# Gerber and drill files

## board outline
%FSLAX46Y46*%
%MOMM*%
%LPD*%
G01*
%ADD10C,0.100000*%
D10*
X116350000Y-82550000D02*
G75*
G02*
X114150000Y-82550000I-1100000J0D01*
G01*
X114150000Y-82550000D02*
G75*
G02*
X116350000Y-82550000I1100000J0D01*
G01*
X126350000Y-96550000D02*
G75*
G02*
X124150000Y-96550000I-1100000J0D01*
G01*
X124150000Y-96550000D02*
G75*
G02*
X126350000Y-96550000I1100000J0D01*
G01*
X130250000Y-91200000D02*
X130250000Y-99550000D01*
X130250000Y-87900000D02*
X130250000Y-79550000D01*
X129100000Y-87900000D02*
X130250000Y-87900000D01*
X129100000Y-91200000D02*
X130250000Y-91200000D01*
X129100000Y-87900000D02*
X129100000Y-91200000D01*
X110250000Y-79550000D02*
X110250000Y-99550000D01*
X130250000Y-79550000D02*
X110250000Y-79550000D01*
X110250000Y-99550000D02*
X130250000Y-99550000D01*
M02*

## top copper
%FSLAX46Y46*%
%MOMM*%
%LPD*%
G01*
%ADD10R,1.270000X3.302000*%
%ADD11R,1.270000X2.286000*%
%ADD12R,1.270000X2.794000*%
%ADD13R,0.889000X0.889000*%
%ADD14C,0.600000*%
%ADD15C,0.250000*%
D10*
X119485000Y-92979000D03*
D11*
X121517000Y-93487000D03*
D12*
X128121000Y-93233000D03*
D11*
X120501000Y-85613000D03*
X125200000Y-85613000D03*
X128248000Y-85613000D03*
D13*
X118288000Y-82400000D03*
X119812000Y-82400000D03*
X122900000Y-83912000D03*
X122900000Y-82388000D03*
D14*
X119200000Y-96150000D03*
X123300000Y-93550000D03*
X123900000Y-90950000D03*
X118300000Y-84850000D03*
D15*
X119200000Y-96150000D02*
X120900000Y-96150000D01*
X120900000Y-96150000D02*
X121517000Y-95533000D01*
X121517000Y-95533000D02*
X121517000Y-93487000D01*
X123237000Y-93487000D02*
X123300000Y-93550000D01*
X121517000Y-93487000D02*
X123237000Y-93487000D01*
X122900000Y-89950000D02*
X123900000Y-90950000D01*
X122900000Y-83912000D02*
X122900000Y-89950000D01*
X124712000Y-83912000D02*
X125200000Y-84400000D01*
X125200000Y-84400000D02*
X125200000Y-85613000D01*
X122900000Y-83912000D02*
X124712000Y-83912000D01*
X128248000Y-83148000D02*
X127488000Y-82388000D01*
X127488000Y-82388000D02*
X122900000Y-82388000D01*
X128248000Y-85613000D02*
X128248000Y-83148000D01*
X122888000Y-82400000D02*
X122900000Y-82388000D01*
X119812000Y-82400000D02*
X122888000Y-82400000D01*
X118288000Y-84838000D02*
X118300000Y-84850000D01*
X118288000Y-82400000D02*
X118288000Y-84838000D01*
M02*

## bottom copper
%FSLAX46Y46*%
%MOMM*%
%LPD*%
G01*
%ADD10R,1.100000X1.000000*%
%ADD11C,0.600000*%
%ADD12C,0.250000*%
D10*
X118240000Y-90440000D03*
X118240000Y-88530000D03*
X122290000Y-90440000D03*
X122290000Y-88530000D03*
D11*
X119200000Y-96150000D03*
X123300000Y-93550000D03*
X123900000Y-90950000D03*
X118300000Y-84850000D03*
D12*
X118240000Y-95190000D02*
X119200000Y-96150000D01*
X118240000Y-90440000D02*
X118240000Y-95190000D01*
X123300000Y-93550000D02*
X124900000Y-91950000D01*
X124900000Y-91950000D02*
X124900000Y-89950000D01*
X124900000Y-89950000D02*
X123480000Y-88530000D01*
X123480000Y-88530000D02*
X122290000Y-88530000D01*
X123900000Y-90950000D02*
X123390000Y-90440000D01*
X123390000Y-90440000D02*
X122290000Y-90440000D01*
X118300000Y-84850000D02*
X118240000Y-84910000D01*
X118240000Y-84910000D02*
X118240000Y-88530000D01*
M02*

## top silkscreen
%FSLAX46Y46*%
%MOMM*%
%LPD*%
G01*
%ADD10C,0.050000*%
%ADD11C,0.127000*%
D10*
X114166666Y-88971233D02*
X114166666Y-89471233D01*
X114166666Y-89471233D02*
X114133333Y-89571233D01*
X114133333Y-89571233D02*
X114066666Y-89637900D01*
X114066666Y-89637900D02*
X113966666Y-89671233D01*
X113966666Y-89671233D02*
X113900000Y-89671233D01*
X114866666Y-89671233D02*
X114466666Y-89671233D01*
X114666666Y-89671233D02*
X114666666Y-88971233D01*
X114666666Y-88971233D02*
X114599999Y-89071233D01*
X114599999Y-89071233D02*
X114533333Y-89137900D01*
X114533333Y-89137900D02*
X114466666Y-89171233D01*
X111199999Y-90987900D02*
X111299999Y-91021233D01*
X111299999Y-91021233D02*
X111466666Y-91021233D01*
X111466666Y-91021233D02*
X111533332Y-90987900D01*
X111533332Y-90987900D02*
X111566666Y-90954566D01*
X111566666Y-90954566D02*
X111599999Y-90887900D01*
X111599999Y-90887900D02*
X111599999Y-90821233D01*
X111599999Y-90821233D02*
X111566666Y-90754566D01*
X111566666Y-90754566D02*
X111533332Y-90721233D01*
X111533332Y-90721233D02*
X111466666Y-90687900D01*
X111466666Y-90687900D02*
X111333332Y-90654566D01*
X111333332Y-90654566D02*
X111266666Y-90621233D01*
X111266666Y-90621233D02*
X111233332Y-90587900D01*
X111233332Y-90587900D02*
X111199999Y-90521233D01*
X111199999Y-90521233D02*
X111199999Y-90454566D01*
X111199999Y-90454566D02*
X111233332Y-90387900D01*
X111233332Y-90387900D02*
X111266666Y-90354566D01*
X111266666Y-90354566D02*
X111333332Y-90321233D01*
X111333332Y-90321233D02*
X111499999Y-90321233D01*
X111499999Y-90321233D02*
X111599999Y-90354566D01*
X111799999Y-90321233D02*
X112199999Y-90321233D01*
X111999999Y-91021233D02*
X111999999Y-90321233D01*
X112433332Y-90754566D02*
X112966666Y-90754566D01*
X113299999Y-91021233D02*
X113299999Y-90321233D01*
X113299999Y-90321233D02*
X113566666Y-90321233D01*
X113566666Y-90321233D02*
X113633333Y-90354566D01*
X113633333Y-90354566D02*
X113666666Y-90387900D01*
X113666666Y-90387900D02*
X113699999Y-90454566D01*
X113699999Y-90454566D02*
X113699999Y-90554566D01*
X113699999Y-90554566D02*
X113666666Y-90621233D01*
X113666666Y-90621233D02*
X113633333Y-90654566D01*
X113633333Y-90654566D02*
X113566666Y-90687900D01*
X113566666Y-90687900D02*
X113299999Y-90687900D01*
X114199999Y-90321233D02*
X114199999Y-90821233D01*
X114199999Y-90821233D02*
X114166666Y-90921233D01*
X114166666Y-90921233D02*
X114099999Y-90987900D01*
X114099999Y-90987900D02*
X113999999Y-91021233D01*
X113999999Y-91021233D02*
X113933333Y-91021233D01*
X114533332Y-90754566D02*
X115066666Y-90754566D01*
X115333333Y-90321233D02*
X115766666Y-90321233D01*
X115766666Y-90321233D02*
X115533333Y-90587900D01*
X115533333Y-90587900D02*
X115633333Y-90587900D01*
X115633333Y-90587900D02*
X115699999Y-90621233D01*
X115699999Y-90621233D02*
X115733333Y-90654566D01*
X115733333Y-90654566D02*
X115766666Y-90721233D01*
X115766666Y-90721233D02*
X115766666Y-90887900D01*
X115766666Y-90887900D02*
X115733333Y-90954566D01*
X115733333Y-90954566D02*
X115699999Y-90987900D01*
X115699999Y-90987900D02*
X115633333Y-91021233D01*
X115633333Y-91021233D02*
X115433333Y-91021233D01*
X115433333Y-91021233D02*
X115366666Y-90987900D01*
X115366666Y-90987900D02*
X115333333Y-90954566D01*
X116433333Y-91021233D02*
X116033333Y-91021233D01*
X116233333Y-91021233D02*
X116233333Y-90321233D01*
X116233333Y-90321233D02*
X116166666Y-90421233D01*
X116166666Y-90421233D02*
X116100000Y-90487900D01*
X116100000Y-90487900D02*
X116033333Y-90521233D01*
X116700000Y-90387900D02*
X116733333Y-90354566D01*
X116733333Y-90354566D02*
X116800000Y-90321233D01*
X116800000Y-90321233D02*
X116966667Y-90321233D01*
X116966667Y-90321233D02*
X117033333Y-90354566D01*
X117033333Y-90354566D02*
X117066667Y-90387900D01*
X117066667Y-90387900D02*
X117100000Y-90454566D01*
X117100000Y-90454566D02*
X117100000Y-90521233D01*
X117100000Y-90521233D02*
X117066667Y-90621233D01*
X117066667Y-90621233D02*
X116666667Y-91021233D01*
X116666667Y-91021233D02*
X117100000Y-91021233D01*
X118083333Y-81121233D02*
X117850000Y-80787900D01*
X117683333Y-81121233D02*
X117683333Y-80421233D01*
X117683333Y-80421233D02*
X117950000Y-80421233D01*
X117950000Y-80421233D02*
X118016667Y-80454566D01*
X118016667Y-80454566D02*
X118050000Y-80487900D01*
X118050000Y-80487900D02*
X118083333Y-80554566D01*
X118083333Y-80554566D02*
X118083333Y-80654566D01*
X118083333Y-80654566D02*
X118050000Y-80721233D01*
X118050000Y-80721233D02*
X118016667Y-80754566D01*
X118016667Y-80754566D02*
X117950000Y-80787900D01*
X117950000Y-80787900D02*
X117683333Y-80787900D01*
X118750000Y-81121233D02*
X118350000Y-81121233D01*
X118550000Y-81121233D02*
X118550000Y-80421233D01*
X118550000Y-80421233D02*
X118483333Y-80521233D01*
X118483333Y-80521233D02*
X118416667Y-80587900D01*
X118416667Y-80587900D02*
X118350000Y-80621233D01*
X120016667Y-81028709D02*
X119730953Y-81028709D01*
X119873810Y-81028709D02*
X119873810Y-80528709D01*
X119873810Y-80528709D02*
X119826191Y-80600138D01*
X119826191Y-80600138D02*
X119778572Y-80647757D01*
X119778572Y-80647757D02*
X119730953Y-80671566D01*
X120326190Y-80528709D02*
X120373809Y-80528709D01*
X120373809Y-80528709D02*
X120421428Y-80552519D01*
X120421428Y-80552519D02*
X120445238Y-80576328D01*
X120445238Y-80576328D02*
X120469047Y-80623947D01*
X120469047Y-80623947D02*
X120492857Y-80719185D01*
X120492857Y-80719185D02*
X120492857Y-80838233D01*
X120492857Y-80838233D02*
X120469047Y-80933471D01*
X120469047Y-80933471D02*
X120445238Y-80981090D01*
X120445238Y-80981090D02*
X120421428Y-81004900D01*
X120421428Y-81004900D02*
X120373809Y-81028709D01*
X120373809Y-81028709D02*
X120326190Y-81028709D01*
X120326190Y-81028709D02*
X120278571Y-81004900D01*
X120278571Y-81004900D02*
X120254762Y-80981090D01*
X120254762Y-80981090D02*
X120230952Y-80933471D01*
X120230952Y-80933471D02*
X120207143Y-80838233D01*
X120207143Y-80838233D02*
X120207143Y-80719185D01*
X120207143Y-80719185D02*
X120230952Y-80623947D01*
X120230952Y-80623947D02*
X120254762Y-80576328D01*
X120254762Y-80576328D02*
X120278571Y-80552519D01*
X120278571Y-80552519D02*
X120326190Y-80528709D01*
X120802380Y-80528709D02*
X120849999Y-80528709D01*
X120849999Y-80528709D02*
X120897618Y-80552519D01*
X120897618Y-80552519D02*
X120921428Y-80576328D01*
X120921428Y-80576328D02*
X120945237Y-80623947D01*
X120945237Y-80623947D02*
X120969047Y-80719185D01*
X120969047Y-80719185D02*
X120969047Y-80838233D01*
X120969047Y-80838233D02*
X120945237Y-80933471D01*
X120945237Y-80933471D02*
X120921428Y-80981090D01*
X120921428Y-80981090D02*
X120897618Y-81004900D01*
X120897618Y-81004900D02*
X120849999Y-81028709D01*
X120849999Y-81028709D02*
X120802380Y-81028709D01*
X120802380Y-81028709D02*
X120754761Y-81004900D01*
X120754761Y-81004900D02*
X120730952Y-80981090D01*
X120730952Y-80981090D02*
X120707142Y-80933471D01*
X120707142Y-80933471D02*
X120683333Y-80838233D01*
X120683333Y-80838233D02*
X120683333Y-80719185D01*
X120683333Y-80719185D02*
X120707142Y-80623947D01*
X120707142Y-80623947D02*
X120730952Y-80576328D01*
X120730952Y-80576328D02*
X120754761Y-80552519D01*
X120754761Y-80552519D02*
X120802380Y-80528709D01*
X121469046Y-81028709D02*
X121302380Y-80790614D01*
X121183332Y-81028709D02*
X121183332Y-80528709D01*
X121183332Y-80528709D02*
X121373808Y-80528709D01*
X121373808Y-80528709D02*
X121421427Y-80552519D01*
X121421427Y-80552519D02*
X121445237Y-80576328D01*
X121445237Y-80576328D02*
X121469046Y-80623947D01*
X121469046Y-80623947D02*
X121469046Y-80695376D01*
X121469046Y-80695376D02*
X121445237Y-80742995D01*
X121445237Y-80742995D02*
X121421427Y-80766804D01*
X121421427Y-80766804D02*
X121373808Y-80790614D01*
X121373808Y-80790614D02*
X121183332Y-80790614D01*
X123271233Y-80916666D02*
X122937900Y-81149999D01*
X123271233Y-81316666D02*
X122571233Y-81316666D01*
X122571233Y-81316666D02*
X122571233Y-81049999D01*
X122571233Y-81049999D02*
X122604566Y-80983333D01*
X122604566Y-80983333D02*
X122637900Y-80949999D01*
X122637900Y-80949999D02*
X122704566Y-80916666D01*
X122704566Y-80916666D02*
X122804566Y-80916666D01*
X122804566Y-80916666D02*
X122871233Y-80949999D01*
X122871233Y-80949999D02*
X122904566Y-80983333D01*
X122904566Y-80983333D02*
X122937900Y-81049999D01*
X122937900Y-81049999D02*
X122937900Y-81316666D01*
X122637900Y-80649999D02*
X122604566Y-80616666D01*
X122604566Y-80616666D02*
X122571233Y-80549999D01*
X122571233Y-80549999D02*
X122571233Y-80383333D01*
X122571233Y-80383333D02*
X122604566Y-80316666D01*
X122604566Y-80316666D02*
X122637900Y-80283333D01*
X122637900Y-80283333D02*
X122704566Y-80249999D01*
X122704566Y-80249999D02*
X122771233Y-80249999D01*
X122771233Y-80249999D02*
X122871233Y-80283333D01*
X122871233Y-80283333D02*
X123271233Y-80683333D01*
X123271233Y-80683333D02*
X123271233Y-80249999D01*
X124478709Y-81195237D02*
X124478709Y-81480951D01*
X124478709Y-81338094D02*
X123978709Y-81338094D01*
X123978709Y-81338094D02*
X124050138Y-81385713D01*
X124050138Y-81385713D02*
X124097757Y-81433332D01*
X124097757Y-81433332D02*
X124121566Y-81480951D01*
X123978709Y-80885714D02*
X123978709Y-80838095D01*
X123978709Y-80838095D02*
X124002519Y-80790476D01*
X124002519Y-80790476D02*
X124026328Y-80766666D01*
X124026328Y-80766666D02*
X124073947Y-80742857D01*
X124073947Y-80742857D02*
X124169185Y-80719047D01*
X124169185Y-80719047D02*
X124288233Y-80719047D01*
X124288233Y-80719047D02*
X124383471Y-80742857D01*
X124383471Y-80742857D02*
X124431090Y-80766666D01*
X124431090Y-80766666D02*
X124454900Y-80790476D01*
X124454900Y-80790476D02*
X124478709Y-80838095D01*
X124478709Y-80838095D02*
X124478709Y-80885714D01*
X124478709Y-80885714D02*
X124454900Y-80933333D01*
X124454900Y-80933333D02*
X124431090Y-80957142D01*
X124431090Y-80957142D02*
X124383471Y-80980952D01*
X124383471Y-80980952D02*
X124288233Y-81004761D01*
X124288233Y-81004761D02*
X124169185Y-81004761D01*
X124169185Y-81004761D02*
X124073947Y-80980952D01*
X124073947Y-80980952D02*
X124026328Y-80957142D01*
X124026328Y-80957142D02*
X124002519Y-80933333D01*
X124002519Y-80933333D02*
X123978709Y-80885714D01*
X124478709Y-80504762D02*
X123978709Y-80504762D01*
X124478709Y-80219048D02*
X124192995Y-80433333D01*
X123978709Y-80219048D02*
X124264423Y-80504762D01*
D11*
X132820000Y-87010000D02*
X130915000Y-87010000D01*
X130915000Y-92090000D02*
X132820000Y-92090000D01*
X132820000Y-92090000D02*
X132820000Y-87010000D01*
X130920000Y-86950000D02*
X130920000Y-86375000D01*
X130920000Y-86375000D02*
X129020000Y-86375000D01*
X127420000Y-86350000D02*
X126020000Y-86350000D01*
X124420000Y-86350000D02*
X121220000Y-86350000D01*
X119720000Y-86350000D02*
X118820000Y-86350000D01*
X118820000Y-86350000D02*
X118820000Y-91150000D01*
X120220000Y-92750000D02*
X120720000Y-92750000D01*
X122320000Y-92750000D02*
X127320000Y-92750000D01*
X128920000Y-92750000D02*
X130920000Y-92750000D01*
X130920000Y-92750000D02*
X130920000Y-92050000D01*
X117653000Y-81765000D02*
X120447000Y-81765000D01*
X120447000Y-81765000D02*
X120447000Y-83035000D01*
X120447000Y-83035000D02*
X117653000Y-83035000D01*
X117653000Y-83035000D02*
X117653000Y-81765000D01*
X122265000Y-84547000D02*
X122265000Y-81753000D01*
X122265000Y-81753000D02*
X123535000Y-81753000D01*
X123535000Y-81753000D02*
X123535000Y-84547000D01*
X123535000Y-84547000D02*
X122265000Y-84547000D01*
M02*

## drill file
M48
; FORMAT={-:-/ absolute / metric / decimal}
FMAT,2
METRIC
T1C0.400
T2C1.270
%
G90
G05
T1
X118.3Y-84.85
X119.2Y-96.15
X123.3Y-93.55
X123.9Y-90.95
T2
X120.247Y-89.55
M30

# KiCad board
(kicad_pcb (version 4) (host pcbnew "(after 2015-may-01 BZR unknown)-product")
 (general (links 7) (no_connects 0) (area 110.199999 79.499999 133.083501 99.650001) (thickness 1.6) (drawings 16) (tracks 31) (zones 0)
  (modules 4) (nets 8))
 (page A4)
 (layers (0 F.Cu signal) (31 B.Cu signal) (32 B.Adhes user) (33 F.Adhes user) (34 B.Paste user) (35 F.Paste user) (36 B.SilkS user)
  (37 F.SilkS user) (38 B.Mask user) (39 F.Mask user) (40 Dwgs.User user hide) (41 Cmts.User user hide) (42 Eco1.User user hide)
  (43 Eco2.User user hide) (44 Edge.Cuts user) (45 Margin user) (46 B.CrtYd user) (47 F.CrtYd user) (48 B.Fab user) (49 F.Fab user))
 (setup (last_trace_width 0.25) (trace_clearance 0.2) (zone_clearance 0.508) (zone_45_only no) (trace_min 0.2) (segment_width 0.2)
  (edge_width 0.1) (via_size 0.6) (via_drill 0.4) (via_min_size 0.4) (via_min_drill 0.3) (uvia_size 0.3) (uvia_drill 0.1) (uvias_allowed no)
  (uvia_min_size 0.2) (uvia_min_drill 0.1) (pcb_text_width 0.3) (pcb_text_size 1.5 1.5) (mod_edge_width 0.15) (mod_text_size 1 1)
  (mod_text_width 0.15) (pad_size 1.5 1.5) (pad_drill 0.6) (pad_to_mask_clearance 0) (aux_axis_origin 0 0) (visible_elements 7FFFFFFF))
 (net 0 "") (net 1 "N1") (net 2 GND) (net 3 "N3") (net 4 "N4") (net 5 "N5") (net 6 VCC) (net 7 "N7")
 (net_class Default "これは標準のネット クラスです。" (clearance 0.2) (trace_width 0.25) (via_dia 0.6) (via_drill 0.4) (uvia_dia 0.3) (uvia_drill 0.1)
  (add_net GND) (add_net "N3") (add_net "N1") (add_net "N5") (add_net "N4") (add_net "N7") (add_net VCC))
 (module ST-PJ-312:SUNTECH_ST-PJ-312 (layer F.Cu) (at 125.2 89.55) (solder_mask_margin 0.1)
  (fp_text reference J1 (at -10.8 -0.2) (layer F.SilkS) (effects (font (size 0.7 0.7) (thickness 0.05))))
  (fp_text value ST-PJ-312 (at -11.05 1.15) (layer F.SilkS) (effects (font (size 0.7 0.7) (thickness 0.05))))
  (fp_line (start 7.62 -2.54) (end 5.715 -2.54) (layer F.SilkS) (width 0.127))
  (fp_line (start 5.715 2.54) (end 7.62 2.54) (layer F.SilkS) (width 0.127))
  (fp_line (start 7.62 2.54) (end 7.62 -2.54) (layer F.SilkS) (width 0.127))
  (fp_line (start 5.72 -2.6) (end 5.72 -3.175) (layer F.SilkS) (width 0.127))
  (fp_line (start 5.72 -3.175) (end 3.82 -3.175) (layer F.SilkS) (width 0.127))
  (fp_line (start 2.22 -3.2) (end 0.82 -3.2) (layer F.SilkS) (width 0.127))
  (fp_line (start -0.78 -3.2) (end -3.98 -3.2) (layer F.SilkS) (width 0.127))
  (fp_line (start -5.48 -3.2) (end -6.38 -3.2) (layer F.SilkS) (width 0.127))
  (fp_line (start -6.38 -3.2) (end -6.38 1.6) (layer F.SilkS) (width 0.127))
  (fp_line (start -4.98 3.2) (end -4.48 3.2) (layer F.SilkS) (width 0.127))
  (fp_line (start -2.88 3.2) (end 2.12 3.2) (layer F.SilkS) (width 0.127))
  (fp_line (start 3.72 3.2) (end 5.72 3.2) (layer F.SilkS) (width 0.127))
  (fp_line (start 5.72 3.2) (end 5.72 2.5) (layer F.SilkS) (width 0.127))
  (pad LS smd rect (at -5.715 3.429 90) (size 3.302 1.27) (layers F.Cu F.Paste F.Mask) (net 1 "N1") (solder_mask_margin 0.2))
  (pad L smd rect (at -3.683 3.937 90) (size 2.286 1.27) (layers F.Cu F.Paste F.Mask) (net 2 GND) (solder_mask_margin 0.2))
  (pad COM2 smd rect (at 2.921 3.683 90) (size 2.794 1.27) (layers F.Cu F.Paste F.Mask) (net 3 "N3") (solder_mask_margin 0.2))
  (pad RS smd rect (at -4.699 -3.937 90) (size 2.286 1.27) (layers F.Cu F.Paste F.Mask) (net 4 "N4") (solder_mask_margin 0.2))
  (pad R smd rect (at 0 -3.937 90) (size 2.286 1.27) (layers F.Cu F.Paste F.Mask) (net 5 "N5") (solder_mask_margin 0.2))
  (pad COM1 smd rect (at 3.048 -3.937 90) (size 2.286 1.27) (layers F.Cu F.Paste F.Mask) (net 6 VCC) (solder_mask_margin 0.2))
  (pad Hole np_thru_hole circle (at -4.953 0) (size 1.27 1.27) (drill 1.27) (layers)))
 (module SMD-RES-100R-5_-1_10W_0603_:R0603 (layer F.Cu) (at 119.05 82.4 90) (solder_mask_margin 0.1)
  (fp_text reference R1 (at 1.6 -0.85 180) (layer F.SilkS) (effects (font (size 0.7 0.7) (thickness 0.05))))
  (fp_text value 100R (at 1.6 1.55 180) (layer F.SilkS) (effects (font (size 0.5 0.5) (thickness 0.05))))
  (fp_line (start 0.635 -1.397) (end 0.635 1.397) (layer F.SilkS) (width 0.127))
  (fp_line (start 0.635 1.397) (end -0.635 1.397) (layer F.SilkS) (width 0.127))
  (fp_line (start -0.635 1.397) (end -0.635 -1.397) (layer F.SilkS) (width 0.127))
  (fp_line (start -0.635 -1.397) (end 0.635 -1.397) (layer F.SilkS) (width 0.127))
  (pad 1 smd rect (at 0 -0.762) (size 0.889 0.889) (layers F.Cu F.Paste F.Mask) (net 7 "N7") (solder_mask_margin 0.2))
  (pad 2 smd rect (at 0 0.762) (size 0.889 0.889) (layers F.Cu F.Paste F.Mask) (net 6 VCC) (solder_mask_margin 0.2)))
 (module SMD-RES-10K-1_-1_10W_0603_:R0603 (layer F.Cu) (at 122.9 83.15 180) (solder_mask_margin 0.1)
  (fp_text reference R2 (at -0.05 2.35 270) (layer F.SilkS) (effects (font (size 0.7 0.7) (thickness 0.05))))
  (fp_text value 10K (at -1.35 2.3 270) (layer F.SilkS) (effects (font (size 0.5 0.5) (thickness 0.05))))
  (fp_line (start 0.635 -1.397) (end 0.635 1.397) (layer F.SilkS) (width 0.127))
  (fp_line (start 0.635 1.397) (end -0.635 1.397) (layer F.SilkS) (width 0.127))
  (fp_line (start -0.635 1.397) (end -0.635 -1.397) (layer F.SilkS) (width 0.127))
  (fp_line (start -0.635 -1.397) (end 0.635 -1.397) (layer F.SilkS) (width 0.127))
  (pad 1 smd rect (at 0 -0.762 90) (size 0.889 0.889) (layers F.Cu F.Paste F.Mask) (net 5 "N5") (solder_mask_margin 0.2))
  (pad 2 smd rect (at 0 0.762 90) (size 0.889 0.889) (layers F.Cu F.Paste F.Mask) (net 6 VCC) (solder_mask_margin 0.2)))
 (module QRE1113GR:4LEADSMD (layer B.Cu) (at 120.25 89.5) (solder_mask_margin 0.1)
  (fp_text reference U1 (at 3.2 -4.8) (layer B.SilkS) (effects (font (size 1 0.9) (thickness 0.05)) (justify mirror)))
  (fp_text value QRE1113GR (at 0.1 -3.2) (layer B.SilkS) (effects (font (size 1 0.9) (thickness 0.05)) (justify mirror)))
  (pad E smd rect (at -2.01 0.94 90) (size 1 1.1) (layers B.Cu B.Paste B.Mask) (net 2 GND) (solder_mask_margin 0.2))
  (pad A smd rect (at -2.01 -0.97 90) (size 1 1.1) (layers B.Cu B.Paste B.Mask) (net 7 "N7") (solder_mask_margin 0.2))
  (pad C smd rect (at 2.04 0.94 90) (size 1 1.1) (layers B.Cu B.Paste B.Mask) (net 5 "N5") (solder_mask_margin 0.2))
  (pad K smd rect (at 2.04 -0.97 90) (size 1 1.1) (layers B.Cu B.Paste B.Mask) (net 2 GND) (solder_mask_margin 0.2)))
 (gr_circle (center 115.25 82.55) (end 116.35 82.55) (layer Edge.Cuts) (width 0.1))
 (gr_circle (center 125.25 96.55) (end 126.35 96.55) (layer Edge.Cuts) (width 0.1))
 (gr_line (start 130.25 91.2) (end 130.25 99.55) (angle 90) (layer Edge.Cuts) (width 0.1))
 (gr_line (start 130.25 87.9) (end 130.25 79.55) (angle 90) (layer Edge.Cuts) (width 0.1))
 (gr_line (start 129.1 87.9) (end 130.25 87.9) (angle 90) (layer Edge.Cuts) (width 0.1))
 (gr_line (start 129.1 91.2) (end 130.25 91.2) (angle 90) (layer Edge.Cuts) (width 0.1))
 (gr_line (start 129.1 87.9) (end 129.1 91.2) (angle 90) (layer Edge.Cuts) (width 0.1))
 (gr_line (start 110.25 79.55) (end 110.25 99.55) (angle 90) (layer Edge.Cuts) (width 0.1))
 (gr_line (start 130.25 79.55) (end 110.25 79.55) (angle 90) (layer Edge.Cuts) (width 0.1))
 (gr_line (start 110.25 99.55) (end 130.25 99.55) (angle 90) (layer Edge.Cuts) (width 0.1))
 (segment (start 118.24 95.19) (end 119.2 96.15) (width 0.25) (layer B.Cu) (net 2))
 (via (at 119.2 96.15) (size 0.6) (layers F.Cu B.Cu) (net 2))
 (segment (start 119.2 96.15) (end 120.9 96.15) (width 0.25) (layer F.Cu) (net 2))
 (segment (start 120.9 96.15) (end 121.517 95.533) (width 0.25) (layer F.Cu) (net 2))
 (segment (start 121.517 95.533) (end 121.517 93.487) (width 0.25) (layer F.Cu) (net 2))
 (segment (start 118.24 90.44) (end 118.24 95.19) (width 0.25) (layer B.Cu) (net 2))
 (segment (start 123.237 93.487) (end 123.3 93.55) (width 0.25) (layer F.Cu) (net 2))
 (via (at 123.3 93.55) (size 0.6) (layers F.Cu B.Cu) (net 2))
 (segment (start 123.3 93.55) (end 124.9 91.95) (width 0.25) (layer B.Cu) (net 2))
 (segment (start 124.9 91.95) (end 124.9 89.95) (width 0.25) (layer B.Cu) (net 2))
 (segment (start 124.9 89.95) (end 123.48 88.53) (width 0.25) (layer B.Cu) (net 2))
 (segment (start 123.48 88.53) (end 122.29 88.53) (width 0.25) (layer B.Cu) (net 2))
 (segment (start 121.517 93.487) (end 123.237 93.487) (width 0.25) (layer F.Cu) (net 2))
 (segment (start 122.9 89.95) (end 123.9 90.95) (width 0.25) (layer F.Cu) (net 5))
 (via (at 123.9 90.95) (size 0.6) (layers F.Cu B.Cu) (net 5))
 (segment (start 123.9 90.95) (end 123.39 90.44) (width 0.25) (layer B.Cu) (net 5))
 (segment (start 123.39 90.44) (end 122.29 90.44) (width 0.25) (layer B.Cu) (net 5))
 (segment (start 122.9 83.912) (end 122.9 89.95) (width 0.25) (layer F.Cu) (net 5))
 (segment (start 124.712 83.912) (end 125.2 84.4) (width 0.25) (layer F.Cu) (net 5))
 (segment (start 125.2 84.4) (end 125.2 85.613) (width 0.25) (layer F.Cu) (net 5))
 (segment (start 122.9 83.912) (end 124.712 83.912) (width 0.25) (layer F.Cu) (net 5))
 (segment (start 128.248 83.148) (end 127.488 82.388) (width 0.25) (layer F.Cu) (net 6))
 (segment (start 127.488 82.388) (end 122.9 82.388) (width 0.25) (layer F.Cu) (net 6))
 (segment (start 128.248 85.613) (end 128.248 83.148) (width 0.25) (layer F.Cu) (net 6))
 (segment (start 122.888 82.4) (end 122.9 82.388) (width 0.25) (layer F.Cu) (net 6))
 (segment (start 119.812 82.4) (end 122.888 82.4) (width 0.25) (layer F.Cu) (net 6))
 (segment (start 118.288 84.838) (end 118.3 84.85) (width 0.25) (layer F.Cu) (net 7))
 (via (at 118.3 84.85) (size 0.6) (layers F.Cu B.Cu) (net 7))
 (segment (start 118.3 84.85) (end 118.24 84.91) (width 0.25) (layer B.Cu) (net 7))
 (segment (start 118.24 84.91) (end 118.24 88.53) (width 0.25) (layer B.Cu) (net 7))
 (segment (start 118.288 82.4) (end 118.288 84.838) (width 0.25) (layer F.Cu) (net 7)))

